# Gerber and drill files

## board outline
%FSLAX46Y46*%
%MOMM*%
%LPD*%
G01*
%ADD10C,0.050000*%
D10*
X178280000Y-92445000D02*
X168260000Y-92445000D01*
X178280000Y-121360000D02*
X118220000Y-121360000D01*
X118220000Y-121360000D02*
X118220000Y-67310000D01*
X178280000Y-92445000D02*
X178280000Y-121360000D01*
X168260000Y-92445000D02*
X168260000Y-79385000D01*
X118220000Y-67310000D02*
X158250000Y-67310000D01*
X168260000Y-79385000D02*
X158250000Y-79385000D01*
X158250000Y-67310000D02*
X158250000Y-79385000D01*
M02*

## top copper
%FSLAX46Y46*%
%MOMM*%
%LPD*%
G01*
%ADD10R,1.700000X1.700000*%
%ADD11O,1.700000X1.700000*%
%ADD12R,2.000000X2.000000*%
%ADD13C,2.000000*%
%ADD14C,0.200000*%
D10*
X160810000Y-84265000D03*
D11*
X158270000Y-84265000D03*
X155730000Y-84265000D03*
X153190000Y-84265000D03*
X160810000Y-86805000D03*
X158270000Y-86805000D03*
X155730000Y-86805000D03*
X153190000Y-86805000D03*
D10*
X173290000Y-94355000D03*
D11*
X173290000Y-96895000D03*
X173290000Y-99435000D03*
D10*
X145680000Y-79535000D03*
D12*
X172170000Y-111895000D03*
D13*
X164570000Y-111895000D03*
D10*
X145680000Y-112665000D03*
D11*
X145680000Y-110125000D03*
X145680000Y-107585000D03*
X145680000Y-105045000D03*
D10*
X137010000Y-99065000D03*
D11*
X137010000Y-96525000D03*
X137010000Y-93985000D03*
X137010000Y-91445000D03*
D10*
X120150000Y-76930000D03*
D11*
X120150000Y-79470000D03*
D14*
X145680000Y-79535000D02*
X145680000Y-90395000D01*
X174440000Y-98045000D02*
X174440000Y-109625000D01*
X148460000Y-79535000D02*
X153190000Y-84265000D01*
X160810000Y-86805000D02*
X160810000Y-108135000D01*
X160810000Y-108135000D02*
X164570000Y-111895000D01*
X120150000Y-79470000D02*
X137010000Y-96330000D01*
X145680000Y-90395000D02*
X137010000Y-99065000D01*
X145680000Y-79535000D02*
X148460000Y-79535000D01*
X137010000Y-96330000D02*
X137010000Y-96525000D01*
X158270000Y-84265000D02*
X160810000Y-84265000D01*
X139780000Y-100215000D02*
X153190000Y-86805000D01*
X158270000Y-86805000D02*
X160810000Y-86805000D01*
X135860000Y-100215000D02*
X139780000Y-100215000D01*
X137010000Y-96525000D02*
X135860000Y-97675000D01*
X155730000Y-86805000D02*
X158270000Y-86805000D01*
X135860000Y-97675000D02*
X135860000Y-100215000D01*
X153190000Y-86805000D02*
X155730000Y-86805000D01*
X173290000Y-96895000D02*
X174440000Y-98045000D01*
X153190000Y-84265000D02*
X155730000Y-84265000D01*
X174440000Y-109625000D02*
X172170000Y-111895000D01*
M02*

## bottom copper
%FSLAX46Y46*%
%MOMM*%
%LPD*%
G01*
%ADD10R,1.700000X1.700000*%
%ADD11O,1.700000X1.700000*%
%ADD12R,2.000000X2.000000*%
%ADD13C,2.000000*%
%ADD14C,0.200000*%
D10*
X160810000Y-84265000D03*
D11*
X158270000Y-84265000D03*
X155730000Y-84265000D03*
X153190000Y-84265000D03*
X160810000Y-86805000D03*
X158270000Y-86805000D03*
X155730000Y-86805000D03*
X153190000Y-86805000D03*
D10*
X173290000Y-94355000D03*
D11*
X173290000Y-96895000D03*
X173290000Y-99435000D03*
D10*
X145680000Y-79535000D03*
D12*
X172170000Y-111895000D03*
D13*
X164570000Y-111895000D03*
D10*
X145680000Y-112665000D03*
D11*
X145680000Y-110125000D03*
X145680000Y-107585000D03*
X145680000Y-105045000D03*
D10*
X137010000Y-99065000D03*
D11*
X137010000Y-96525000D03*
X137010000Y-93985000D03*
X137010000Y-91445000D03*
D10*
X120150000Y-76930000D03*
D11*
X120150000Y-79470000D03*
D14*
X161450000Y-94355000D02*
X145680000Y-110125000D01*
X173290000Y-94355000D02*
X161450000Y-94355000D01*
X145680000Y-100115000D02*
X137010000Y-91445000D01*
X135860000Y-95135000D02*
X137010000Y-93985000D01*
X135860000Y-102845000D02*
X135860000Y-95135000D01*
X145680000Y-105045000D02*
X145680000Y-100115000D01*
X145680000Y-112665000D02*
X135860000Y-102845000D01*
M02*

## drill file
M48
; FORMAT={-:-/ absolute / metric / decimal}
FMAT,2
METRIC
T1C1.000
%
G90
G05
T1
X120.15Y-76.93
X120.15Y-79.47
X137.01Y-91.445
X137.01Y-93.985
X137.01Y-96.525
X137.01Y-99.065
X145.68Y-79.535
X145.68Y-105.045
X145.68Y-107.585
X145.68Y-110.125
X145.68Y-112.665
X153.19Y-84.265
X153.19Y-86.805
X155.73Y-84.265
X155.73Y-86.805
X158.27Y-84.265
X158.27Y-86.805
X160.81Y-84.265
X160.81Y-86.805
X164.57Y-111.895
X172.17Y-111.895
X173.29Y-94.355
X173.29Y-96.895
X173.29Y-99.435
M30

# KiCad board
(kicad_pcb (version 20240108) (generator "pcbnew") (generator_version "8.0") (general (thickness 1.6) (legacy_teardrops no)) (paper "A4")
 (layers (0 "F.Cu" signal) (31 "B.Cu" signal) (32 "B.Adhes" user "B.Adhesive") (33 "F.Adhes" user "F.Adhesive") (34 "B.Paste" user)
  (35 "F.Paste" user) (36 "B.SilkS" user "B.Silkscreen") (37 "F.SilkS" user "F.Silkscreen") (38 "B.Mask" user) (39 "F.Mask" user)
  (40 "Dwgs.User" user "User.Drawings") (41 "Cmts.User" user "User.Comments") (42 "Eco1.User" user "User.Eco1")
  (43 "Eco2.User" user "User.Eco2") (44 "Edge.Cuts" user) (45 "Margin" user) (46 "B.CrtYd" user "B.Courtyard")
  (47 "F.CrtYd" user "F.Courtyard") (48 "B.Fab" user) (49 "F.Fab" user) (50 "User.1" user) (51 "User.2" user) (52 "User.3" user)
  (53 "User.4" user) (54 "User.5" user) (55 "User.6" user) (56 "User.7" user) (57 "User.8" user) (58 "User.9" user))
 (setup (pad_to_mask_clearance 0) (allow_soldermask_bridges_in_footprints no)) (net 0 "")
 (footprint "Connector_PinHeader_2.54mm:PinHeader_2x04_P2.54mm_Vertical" (layer "F.Cu") (at 160.81 84.265 -90)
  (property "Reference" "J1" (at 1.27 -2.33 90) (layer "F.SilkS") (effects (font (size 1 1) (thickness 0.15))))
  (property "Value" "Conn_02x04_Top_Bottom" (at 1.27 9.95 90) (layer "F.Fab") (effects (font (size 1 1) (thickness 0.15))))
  (pad "1" thru_hole rect (at 0 0 270) (size 1.7 1.7) (drill 1) (layers "*.Cu" "*.Mask") (remove_unused_layers no))
  (pad "2" thru_hole oval (at 0 2.54 270) (size 1.7 1.7) (drill 1) (layers "*.Cu" "*.Mask") (remove_unused_layers no))
  (pad "3" thru_hole oval (at 0 5.08 270) (size 1.7 1.7) (drill 1) (layers "*.Cu" "*.Mask") (remove_unused_layers no))
  (pad "4" thru_hole oval (at 0 7.62 270) (size 1.7 1.7) (drill 1) (layers "*.Cu" "*.Mask") (remove_unused_layers no))
  (pad "5" thru_hole oval (at 2.54 0 270) (size 1.7 1.7) (drill 1) (layers "*.Cu" "*.Mask") (remove_unused_layers no))
  (pad "6" thru_hole oval (at 2.54 2.54 270) (size 1.7 1.7) (drill 1) (layers "*.Cu" "*.Mask") (remove_unused_layers no))
  (pad "7" thru_hole oval (at 2.54 5.08 270) (size 1.7 1.7) (drill 1) (layers "*.Cu" "*.Mask") (remove_unused_layers no))
  (pad "8" thru_hole oval (at 2.54 7.62 270) (size 1.7 1.7) (drill 1) (layers "*.Cu" "*.Mask") (remove_unused_layers no)))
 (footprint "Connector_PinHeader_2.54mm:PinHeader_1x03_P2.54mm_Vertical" (layer "F.Cu") (at 173.29 94.355)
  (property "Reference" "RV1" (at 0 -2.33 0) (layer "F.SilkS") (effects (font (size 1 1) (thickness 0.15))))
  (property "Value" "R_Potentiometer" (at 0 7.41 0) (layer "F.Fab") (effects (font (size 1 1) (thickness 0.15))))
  (pad "1" thru_hole rect (at 0 0) (size 1.7 1.7) (drill 1) (layers "*.Cu" "*.Mask") (remove_unused_layers no))
  (pad "2" thru_hole oval (at 0 2.54) (size 1.7 1.7) (drill 1) (layers "*.Cu" "*.Mask") (remove_unused_layers no))
  (pad "3" thru_hole oval (at 0 5.08) (size 1.7 1.7) (drill 1) (layers "*.Cu" "*.Mask") (remove_unused_layers no)))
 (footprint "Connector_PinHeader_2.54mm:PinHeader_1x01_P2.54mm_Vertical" (layer "F.Cu") (at 145.68 79.535)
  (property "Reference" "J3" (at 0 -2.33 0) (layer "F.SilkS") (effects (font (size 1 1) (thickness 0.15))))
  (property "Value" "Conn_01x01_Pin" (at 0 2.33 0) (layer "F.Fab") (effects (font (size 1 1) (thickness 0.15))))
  (pad "1" thru_hole rect (at 0 0) (size 1.7 1.7) (drill 1) (layers "*.Cu" "*.Mask") (remove_unused_layers no)))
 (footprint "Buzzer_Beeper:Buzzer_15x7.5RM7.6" (layer "F.Cu") (at 172.17 111.895 180)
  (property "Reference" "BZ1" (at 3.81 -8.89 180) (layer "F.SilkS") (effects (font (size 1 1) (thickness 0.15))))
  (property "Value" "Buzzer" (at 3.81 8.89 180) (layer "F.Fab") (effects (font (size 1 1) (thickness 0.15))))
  (pad "1" thru_hole rect (at 0 0 180) (size 2 2) (drill 1) (layers "*.Cu" "*.Mask") (remove_unused_layers no))
  (pad "2" thru_hole circle (at 7.6 0 180) (size 2 2) (drill 1) (layers "*.Cu" "*.Mask") (remove_unused_layers no)))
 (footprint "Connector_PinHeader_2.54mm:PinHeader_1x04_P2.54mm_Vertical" (layer "F.Cu") (at 145.68 112.665 180)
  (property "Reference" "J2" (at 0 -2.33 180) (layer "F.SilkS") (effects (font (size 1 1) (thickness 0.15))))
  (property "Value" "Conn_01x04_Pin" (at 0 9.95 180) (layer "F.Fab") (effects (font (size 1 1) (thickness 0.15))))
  (pad "1" thru_hole rect (at 0 0 180) (size 1.7 1.7) (drill 1) (layers "*.Cu" "*.Mask") (remove_unused_layers no))
  (pad "2" thru_hole oval (at 0 2.54 180) (size 1.7 1.7) (drill 1) (layers "*.Cu" "*.Mask") (remove_unused_layers no))
  (pad "3" thru_hole oval (at 0 5.08 180) (size 1.7 1.7) (drill 1) (layers "*.Cu" "*.Mask") (remove_unused_layers no))
  (pad "4" thru_hole oval (at 0 7.62 180) (size 1.7 1.7) (drill 1) (layers "*.Cu" "*.Mask") (remove_unused_layers no)))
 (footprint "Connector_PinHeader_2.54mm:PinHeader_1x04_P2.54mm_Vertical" (layer "F.Cu") (at 137.01 99.065 180)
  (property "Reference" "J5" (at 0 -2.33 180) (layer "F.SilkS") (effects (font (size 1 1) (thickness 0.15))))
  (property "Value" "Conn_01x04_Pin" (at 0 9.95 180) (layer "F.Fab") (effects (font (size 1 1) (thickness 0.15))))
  (pad "1" thru_hole rect (at 0 0 180) (size 1.7 1.7) (drill 1) (layers "*.Cu" "*.Mask") (remove_unused_layers no))
  (pad "2" thru_hole oval (at 0 2.54 180) (size 1.7 1.7) (drill 1) (layers "*.Cu" "*.Mask") (remove_unused_layers no))
  (pad "3" thru_hole oval (at 0 5.08 180) (size 1.7 1.7) (drill 1) (layers "*.Cu" "*.Mask") (remove_unused_layers no))
  (pad "4" thru_hole oval (at 0 7.62 180) (size 1.7 1.7) (drill 1) (layers "*.Cu" "*.Mask") (remove_unused_layers no)))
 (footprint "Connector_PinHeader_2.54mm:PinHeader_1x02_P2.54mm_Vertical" (layer "F.Cu") (at 120.15 76.93)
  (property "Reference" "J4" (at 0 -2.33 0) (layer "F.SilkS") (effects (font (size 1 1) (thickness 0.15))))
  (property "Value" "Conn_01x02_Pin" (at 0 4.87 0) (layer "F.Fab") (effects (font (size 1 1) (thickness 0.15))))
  (pad "1" thru_hole rect (at 0 0) (size 1.7 1.7) (drill 1) (layers "*.Cu" "*.Mask") (remove_unused_layers no))
  (pad "2" thru_hole oval (at 0 2.54) (size 1.7 1.7) (drill 1) (layers "*.Cu" "*.Mask") (remove_unused_layers no)))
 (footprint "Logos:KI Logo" (layer "F.Cu") (at 144.664834 101.475)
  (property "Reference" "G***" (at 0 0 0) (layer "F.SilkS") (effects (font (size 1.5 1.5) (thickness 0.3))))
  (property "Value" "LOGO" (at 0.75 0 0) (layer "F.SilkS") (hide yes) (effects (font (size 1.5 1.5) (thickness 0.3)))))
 (gr_line (start 178.28 92.445) (end 168.26 92.445) (stroke (width 0.05) (type default)) (layer "Edge.Cuts"))
 (gr_line (start 178.28 121.36) (end 118.22 121.36) (stroke (width 0.05) (type default)) (layer "Edge.Cuts"))
 (gr_line (start 118.22 121.36) (end 118.22 67.31) (stroke (width 0.05) (type default)) (layer "Edge.Cuts"))
 (gr_line (start 178.28 92.445) (end 178.28 121.36) (stroke (width 0.05) (type default)) (layer "Edge.Cuts"))
 (gr_line (start 168.26 92.445) (end 168.26 79.385) (stroke (width 0.05) (type default)) (layer "Edge.Cuts"))
 (gr_line (start 118.22 67.31) (end 158.25 67.31) (stroke (width 0.05) (type default)) (layer "Edge.Cuts"))
 (gr_line (start 168.26 79.385) (end 158.25 79.385) (stroke (width 0.05) (type default)) (layer "Edge.Cuts"))
 (gr_line (start 158.25 67.31) (end 158.25 79.385) (stroke (width 0.05) (type default)) (layer "Edge.Cuts"))
 (segment (start 145.68 79.535) (end 145.68 90.395) (width 0.2) (layer "F.Cu") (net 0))
 (segment (start 174.44 98.045) (end 174.44 109.625) (width 0.2) (layer "F.Cu") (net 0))
 (segment (start 148.46 79.535) (end 153.19 84.265) (width 0.2) (layer "F.Cu") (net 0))
 (segment (start 160.81 86.805) (end 160.81 108.135) (width 0.2) (layer "F.Cu") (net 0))
 (segment (start 160.81 108.135) (end 164.57 111.895) (width 0.2) (layer "F.Cu") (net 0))
 (segment (start 120.15 79.47) (end 137.01 96.33) (width 0.2) (layer "F.Cu") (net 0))
 (segment (start 145.68 90.395) (end 137.01 99.065) (width 0.2) (layer "F.Cu") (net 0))
 (segment (start 145.68 79.535) (end 148.46 79.535) (width 0.2) (layer "F.Cu") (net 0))
 (segment (start 137.01 96.33) (end 137.01 96.525) (width 0.2) (layer "F.Cu") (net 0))
 (segment (start 158.27 84.265) (end 160.81 84.265) (width 0.2) (layer "F.Cu") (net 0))
 (segment (start 139.78 100.215) (end 153.19 86.805) (width 0.2) (layer "F.Cu") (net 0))
 (segment (start 158.27 86.805) (end 160.81 86.805) (width 0.2) (layer "F.Cu") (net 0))
 (segment (start 135.86 100.215) (end 139.78 100.215) (width 0.2) (layer "F.Cu") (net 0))
 (segment (start 137.01 96.525) (end 135.86 97.675) (width 0.2) (layer "F.Cu") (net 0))
 (segment (start 155.73 86.805) (end 158.27 86.805) (width 0.2) (layer "F.Cu") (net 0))
 (segment (start 135.86 97.675) (end 135.86 100.215) (width 0.2) (layer "F.Cu") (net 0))
 (segment (start 153.19 86.805) (end 155.73 86.805) (width 0.2) (layer "F.Cu") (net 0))
 (segment (start 173.29 96.895) (end 174.44 98.045) (width 0.2) (layer "F.Cu") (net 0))
 (segment (start 153.19 84.265) (end 155.73 84.265) (width 0.2) (layer "F.Cu") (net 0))
 (segment (start 174.44 109.625) (end 172.17 111.895) (width 0.2) (layer "F.Cu") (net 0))
 (segment (start 161.45 94.355) (end 145.68 110.125) (width 0.2) (layer "B.Cu") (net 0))
 (segment (start 173.29 94.355) (end 161.45 94.355) (width 0.2) (layer "B.Cu") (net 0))
 (segment (start 145.68 100.115) (end 137.01 91.445) (width 0.2) (layer "B.Cu") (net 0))
 (segment (start 135.86 95.135) (end 137.01 93.985) (width 0.2) (layer "B.Cu") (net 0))
 (segment (start 135.86 102.845) (end 135.86 95.135) (width 0.2) (layer "B.Cu") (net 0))
 (segment (start 145.68 105.045) (end 145.68 100.115) (width 0.2) (layer "B.Cu") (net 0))
 (segment (start 145.68 112.665) (end 135.86 102.845) (width 0.2) (layer "B.Cu") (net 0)))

